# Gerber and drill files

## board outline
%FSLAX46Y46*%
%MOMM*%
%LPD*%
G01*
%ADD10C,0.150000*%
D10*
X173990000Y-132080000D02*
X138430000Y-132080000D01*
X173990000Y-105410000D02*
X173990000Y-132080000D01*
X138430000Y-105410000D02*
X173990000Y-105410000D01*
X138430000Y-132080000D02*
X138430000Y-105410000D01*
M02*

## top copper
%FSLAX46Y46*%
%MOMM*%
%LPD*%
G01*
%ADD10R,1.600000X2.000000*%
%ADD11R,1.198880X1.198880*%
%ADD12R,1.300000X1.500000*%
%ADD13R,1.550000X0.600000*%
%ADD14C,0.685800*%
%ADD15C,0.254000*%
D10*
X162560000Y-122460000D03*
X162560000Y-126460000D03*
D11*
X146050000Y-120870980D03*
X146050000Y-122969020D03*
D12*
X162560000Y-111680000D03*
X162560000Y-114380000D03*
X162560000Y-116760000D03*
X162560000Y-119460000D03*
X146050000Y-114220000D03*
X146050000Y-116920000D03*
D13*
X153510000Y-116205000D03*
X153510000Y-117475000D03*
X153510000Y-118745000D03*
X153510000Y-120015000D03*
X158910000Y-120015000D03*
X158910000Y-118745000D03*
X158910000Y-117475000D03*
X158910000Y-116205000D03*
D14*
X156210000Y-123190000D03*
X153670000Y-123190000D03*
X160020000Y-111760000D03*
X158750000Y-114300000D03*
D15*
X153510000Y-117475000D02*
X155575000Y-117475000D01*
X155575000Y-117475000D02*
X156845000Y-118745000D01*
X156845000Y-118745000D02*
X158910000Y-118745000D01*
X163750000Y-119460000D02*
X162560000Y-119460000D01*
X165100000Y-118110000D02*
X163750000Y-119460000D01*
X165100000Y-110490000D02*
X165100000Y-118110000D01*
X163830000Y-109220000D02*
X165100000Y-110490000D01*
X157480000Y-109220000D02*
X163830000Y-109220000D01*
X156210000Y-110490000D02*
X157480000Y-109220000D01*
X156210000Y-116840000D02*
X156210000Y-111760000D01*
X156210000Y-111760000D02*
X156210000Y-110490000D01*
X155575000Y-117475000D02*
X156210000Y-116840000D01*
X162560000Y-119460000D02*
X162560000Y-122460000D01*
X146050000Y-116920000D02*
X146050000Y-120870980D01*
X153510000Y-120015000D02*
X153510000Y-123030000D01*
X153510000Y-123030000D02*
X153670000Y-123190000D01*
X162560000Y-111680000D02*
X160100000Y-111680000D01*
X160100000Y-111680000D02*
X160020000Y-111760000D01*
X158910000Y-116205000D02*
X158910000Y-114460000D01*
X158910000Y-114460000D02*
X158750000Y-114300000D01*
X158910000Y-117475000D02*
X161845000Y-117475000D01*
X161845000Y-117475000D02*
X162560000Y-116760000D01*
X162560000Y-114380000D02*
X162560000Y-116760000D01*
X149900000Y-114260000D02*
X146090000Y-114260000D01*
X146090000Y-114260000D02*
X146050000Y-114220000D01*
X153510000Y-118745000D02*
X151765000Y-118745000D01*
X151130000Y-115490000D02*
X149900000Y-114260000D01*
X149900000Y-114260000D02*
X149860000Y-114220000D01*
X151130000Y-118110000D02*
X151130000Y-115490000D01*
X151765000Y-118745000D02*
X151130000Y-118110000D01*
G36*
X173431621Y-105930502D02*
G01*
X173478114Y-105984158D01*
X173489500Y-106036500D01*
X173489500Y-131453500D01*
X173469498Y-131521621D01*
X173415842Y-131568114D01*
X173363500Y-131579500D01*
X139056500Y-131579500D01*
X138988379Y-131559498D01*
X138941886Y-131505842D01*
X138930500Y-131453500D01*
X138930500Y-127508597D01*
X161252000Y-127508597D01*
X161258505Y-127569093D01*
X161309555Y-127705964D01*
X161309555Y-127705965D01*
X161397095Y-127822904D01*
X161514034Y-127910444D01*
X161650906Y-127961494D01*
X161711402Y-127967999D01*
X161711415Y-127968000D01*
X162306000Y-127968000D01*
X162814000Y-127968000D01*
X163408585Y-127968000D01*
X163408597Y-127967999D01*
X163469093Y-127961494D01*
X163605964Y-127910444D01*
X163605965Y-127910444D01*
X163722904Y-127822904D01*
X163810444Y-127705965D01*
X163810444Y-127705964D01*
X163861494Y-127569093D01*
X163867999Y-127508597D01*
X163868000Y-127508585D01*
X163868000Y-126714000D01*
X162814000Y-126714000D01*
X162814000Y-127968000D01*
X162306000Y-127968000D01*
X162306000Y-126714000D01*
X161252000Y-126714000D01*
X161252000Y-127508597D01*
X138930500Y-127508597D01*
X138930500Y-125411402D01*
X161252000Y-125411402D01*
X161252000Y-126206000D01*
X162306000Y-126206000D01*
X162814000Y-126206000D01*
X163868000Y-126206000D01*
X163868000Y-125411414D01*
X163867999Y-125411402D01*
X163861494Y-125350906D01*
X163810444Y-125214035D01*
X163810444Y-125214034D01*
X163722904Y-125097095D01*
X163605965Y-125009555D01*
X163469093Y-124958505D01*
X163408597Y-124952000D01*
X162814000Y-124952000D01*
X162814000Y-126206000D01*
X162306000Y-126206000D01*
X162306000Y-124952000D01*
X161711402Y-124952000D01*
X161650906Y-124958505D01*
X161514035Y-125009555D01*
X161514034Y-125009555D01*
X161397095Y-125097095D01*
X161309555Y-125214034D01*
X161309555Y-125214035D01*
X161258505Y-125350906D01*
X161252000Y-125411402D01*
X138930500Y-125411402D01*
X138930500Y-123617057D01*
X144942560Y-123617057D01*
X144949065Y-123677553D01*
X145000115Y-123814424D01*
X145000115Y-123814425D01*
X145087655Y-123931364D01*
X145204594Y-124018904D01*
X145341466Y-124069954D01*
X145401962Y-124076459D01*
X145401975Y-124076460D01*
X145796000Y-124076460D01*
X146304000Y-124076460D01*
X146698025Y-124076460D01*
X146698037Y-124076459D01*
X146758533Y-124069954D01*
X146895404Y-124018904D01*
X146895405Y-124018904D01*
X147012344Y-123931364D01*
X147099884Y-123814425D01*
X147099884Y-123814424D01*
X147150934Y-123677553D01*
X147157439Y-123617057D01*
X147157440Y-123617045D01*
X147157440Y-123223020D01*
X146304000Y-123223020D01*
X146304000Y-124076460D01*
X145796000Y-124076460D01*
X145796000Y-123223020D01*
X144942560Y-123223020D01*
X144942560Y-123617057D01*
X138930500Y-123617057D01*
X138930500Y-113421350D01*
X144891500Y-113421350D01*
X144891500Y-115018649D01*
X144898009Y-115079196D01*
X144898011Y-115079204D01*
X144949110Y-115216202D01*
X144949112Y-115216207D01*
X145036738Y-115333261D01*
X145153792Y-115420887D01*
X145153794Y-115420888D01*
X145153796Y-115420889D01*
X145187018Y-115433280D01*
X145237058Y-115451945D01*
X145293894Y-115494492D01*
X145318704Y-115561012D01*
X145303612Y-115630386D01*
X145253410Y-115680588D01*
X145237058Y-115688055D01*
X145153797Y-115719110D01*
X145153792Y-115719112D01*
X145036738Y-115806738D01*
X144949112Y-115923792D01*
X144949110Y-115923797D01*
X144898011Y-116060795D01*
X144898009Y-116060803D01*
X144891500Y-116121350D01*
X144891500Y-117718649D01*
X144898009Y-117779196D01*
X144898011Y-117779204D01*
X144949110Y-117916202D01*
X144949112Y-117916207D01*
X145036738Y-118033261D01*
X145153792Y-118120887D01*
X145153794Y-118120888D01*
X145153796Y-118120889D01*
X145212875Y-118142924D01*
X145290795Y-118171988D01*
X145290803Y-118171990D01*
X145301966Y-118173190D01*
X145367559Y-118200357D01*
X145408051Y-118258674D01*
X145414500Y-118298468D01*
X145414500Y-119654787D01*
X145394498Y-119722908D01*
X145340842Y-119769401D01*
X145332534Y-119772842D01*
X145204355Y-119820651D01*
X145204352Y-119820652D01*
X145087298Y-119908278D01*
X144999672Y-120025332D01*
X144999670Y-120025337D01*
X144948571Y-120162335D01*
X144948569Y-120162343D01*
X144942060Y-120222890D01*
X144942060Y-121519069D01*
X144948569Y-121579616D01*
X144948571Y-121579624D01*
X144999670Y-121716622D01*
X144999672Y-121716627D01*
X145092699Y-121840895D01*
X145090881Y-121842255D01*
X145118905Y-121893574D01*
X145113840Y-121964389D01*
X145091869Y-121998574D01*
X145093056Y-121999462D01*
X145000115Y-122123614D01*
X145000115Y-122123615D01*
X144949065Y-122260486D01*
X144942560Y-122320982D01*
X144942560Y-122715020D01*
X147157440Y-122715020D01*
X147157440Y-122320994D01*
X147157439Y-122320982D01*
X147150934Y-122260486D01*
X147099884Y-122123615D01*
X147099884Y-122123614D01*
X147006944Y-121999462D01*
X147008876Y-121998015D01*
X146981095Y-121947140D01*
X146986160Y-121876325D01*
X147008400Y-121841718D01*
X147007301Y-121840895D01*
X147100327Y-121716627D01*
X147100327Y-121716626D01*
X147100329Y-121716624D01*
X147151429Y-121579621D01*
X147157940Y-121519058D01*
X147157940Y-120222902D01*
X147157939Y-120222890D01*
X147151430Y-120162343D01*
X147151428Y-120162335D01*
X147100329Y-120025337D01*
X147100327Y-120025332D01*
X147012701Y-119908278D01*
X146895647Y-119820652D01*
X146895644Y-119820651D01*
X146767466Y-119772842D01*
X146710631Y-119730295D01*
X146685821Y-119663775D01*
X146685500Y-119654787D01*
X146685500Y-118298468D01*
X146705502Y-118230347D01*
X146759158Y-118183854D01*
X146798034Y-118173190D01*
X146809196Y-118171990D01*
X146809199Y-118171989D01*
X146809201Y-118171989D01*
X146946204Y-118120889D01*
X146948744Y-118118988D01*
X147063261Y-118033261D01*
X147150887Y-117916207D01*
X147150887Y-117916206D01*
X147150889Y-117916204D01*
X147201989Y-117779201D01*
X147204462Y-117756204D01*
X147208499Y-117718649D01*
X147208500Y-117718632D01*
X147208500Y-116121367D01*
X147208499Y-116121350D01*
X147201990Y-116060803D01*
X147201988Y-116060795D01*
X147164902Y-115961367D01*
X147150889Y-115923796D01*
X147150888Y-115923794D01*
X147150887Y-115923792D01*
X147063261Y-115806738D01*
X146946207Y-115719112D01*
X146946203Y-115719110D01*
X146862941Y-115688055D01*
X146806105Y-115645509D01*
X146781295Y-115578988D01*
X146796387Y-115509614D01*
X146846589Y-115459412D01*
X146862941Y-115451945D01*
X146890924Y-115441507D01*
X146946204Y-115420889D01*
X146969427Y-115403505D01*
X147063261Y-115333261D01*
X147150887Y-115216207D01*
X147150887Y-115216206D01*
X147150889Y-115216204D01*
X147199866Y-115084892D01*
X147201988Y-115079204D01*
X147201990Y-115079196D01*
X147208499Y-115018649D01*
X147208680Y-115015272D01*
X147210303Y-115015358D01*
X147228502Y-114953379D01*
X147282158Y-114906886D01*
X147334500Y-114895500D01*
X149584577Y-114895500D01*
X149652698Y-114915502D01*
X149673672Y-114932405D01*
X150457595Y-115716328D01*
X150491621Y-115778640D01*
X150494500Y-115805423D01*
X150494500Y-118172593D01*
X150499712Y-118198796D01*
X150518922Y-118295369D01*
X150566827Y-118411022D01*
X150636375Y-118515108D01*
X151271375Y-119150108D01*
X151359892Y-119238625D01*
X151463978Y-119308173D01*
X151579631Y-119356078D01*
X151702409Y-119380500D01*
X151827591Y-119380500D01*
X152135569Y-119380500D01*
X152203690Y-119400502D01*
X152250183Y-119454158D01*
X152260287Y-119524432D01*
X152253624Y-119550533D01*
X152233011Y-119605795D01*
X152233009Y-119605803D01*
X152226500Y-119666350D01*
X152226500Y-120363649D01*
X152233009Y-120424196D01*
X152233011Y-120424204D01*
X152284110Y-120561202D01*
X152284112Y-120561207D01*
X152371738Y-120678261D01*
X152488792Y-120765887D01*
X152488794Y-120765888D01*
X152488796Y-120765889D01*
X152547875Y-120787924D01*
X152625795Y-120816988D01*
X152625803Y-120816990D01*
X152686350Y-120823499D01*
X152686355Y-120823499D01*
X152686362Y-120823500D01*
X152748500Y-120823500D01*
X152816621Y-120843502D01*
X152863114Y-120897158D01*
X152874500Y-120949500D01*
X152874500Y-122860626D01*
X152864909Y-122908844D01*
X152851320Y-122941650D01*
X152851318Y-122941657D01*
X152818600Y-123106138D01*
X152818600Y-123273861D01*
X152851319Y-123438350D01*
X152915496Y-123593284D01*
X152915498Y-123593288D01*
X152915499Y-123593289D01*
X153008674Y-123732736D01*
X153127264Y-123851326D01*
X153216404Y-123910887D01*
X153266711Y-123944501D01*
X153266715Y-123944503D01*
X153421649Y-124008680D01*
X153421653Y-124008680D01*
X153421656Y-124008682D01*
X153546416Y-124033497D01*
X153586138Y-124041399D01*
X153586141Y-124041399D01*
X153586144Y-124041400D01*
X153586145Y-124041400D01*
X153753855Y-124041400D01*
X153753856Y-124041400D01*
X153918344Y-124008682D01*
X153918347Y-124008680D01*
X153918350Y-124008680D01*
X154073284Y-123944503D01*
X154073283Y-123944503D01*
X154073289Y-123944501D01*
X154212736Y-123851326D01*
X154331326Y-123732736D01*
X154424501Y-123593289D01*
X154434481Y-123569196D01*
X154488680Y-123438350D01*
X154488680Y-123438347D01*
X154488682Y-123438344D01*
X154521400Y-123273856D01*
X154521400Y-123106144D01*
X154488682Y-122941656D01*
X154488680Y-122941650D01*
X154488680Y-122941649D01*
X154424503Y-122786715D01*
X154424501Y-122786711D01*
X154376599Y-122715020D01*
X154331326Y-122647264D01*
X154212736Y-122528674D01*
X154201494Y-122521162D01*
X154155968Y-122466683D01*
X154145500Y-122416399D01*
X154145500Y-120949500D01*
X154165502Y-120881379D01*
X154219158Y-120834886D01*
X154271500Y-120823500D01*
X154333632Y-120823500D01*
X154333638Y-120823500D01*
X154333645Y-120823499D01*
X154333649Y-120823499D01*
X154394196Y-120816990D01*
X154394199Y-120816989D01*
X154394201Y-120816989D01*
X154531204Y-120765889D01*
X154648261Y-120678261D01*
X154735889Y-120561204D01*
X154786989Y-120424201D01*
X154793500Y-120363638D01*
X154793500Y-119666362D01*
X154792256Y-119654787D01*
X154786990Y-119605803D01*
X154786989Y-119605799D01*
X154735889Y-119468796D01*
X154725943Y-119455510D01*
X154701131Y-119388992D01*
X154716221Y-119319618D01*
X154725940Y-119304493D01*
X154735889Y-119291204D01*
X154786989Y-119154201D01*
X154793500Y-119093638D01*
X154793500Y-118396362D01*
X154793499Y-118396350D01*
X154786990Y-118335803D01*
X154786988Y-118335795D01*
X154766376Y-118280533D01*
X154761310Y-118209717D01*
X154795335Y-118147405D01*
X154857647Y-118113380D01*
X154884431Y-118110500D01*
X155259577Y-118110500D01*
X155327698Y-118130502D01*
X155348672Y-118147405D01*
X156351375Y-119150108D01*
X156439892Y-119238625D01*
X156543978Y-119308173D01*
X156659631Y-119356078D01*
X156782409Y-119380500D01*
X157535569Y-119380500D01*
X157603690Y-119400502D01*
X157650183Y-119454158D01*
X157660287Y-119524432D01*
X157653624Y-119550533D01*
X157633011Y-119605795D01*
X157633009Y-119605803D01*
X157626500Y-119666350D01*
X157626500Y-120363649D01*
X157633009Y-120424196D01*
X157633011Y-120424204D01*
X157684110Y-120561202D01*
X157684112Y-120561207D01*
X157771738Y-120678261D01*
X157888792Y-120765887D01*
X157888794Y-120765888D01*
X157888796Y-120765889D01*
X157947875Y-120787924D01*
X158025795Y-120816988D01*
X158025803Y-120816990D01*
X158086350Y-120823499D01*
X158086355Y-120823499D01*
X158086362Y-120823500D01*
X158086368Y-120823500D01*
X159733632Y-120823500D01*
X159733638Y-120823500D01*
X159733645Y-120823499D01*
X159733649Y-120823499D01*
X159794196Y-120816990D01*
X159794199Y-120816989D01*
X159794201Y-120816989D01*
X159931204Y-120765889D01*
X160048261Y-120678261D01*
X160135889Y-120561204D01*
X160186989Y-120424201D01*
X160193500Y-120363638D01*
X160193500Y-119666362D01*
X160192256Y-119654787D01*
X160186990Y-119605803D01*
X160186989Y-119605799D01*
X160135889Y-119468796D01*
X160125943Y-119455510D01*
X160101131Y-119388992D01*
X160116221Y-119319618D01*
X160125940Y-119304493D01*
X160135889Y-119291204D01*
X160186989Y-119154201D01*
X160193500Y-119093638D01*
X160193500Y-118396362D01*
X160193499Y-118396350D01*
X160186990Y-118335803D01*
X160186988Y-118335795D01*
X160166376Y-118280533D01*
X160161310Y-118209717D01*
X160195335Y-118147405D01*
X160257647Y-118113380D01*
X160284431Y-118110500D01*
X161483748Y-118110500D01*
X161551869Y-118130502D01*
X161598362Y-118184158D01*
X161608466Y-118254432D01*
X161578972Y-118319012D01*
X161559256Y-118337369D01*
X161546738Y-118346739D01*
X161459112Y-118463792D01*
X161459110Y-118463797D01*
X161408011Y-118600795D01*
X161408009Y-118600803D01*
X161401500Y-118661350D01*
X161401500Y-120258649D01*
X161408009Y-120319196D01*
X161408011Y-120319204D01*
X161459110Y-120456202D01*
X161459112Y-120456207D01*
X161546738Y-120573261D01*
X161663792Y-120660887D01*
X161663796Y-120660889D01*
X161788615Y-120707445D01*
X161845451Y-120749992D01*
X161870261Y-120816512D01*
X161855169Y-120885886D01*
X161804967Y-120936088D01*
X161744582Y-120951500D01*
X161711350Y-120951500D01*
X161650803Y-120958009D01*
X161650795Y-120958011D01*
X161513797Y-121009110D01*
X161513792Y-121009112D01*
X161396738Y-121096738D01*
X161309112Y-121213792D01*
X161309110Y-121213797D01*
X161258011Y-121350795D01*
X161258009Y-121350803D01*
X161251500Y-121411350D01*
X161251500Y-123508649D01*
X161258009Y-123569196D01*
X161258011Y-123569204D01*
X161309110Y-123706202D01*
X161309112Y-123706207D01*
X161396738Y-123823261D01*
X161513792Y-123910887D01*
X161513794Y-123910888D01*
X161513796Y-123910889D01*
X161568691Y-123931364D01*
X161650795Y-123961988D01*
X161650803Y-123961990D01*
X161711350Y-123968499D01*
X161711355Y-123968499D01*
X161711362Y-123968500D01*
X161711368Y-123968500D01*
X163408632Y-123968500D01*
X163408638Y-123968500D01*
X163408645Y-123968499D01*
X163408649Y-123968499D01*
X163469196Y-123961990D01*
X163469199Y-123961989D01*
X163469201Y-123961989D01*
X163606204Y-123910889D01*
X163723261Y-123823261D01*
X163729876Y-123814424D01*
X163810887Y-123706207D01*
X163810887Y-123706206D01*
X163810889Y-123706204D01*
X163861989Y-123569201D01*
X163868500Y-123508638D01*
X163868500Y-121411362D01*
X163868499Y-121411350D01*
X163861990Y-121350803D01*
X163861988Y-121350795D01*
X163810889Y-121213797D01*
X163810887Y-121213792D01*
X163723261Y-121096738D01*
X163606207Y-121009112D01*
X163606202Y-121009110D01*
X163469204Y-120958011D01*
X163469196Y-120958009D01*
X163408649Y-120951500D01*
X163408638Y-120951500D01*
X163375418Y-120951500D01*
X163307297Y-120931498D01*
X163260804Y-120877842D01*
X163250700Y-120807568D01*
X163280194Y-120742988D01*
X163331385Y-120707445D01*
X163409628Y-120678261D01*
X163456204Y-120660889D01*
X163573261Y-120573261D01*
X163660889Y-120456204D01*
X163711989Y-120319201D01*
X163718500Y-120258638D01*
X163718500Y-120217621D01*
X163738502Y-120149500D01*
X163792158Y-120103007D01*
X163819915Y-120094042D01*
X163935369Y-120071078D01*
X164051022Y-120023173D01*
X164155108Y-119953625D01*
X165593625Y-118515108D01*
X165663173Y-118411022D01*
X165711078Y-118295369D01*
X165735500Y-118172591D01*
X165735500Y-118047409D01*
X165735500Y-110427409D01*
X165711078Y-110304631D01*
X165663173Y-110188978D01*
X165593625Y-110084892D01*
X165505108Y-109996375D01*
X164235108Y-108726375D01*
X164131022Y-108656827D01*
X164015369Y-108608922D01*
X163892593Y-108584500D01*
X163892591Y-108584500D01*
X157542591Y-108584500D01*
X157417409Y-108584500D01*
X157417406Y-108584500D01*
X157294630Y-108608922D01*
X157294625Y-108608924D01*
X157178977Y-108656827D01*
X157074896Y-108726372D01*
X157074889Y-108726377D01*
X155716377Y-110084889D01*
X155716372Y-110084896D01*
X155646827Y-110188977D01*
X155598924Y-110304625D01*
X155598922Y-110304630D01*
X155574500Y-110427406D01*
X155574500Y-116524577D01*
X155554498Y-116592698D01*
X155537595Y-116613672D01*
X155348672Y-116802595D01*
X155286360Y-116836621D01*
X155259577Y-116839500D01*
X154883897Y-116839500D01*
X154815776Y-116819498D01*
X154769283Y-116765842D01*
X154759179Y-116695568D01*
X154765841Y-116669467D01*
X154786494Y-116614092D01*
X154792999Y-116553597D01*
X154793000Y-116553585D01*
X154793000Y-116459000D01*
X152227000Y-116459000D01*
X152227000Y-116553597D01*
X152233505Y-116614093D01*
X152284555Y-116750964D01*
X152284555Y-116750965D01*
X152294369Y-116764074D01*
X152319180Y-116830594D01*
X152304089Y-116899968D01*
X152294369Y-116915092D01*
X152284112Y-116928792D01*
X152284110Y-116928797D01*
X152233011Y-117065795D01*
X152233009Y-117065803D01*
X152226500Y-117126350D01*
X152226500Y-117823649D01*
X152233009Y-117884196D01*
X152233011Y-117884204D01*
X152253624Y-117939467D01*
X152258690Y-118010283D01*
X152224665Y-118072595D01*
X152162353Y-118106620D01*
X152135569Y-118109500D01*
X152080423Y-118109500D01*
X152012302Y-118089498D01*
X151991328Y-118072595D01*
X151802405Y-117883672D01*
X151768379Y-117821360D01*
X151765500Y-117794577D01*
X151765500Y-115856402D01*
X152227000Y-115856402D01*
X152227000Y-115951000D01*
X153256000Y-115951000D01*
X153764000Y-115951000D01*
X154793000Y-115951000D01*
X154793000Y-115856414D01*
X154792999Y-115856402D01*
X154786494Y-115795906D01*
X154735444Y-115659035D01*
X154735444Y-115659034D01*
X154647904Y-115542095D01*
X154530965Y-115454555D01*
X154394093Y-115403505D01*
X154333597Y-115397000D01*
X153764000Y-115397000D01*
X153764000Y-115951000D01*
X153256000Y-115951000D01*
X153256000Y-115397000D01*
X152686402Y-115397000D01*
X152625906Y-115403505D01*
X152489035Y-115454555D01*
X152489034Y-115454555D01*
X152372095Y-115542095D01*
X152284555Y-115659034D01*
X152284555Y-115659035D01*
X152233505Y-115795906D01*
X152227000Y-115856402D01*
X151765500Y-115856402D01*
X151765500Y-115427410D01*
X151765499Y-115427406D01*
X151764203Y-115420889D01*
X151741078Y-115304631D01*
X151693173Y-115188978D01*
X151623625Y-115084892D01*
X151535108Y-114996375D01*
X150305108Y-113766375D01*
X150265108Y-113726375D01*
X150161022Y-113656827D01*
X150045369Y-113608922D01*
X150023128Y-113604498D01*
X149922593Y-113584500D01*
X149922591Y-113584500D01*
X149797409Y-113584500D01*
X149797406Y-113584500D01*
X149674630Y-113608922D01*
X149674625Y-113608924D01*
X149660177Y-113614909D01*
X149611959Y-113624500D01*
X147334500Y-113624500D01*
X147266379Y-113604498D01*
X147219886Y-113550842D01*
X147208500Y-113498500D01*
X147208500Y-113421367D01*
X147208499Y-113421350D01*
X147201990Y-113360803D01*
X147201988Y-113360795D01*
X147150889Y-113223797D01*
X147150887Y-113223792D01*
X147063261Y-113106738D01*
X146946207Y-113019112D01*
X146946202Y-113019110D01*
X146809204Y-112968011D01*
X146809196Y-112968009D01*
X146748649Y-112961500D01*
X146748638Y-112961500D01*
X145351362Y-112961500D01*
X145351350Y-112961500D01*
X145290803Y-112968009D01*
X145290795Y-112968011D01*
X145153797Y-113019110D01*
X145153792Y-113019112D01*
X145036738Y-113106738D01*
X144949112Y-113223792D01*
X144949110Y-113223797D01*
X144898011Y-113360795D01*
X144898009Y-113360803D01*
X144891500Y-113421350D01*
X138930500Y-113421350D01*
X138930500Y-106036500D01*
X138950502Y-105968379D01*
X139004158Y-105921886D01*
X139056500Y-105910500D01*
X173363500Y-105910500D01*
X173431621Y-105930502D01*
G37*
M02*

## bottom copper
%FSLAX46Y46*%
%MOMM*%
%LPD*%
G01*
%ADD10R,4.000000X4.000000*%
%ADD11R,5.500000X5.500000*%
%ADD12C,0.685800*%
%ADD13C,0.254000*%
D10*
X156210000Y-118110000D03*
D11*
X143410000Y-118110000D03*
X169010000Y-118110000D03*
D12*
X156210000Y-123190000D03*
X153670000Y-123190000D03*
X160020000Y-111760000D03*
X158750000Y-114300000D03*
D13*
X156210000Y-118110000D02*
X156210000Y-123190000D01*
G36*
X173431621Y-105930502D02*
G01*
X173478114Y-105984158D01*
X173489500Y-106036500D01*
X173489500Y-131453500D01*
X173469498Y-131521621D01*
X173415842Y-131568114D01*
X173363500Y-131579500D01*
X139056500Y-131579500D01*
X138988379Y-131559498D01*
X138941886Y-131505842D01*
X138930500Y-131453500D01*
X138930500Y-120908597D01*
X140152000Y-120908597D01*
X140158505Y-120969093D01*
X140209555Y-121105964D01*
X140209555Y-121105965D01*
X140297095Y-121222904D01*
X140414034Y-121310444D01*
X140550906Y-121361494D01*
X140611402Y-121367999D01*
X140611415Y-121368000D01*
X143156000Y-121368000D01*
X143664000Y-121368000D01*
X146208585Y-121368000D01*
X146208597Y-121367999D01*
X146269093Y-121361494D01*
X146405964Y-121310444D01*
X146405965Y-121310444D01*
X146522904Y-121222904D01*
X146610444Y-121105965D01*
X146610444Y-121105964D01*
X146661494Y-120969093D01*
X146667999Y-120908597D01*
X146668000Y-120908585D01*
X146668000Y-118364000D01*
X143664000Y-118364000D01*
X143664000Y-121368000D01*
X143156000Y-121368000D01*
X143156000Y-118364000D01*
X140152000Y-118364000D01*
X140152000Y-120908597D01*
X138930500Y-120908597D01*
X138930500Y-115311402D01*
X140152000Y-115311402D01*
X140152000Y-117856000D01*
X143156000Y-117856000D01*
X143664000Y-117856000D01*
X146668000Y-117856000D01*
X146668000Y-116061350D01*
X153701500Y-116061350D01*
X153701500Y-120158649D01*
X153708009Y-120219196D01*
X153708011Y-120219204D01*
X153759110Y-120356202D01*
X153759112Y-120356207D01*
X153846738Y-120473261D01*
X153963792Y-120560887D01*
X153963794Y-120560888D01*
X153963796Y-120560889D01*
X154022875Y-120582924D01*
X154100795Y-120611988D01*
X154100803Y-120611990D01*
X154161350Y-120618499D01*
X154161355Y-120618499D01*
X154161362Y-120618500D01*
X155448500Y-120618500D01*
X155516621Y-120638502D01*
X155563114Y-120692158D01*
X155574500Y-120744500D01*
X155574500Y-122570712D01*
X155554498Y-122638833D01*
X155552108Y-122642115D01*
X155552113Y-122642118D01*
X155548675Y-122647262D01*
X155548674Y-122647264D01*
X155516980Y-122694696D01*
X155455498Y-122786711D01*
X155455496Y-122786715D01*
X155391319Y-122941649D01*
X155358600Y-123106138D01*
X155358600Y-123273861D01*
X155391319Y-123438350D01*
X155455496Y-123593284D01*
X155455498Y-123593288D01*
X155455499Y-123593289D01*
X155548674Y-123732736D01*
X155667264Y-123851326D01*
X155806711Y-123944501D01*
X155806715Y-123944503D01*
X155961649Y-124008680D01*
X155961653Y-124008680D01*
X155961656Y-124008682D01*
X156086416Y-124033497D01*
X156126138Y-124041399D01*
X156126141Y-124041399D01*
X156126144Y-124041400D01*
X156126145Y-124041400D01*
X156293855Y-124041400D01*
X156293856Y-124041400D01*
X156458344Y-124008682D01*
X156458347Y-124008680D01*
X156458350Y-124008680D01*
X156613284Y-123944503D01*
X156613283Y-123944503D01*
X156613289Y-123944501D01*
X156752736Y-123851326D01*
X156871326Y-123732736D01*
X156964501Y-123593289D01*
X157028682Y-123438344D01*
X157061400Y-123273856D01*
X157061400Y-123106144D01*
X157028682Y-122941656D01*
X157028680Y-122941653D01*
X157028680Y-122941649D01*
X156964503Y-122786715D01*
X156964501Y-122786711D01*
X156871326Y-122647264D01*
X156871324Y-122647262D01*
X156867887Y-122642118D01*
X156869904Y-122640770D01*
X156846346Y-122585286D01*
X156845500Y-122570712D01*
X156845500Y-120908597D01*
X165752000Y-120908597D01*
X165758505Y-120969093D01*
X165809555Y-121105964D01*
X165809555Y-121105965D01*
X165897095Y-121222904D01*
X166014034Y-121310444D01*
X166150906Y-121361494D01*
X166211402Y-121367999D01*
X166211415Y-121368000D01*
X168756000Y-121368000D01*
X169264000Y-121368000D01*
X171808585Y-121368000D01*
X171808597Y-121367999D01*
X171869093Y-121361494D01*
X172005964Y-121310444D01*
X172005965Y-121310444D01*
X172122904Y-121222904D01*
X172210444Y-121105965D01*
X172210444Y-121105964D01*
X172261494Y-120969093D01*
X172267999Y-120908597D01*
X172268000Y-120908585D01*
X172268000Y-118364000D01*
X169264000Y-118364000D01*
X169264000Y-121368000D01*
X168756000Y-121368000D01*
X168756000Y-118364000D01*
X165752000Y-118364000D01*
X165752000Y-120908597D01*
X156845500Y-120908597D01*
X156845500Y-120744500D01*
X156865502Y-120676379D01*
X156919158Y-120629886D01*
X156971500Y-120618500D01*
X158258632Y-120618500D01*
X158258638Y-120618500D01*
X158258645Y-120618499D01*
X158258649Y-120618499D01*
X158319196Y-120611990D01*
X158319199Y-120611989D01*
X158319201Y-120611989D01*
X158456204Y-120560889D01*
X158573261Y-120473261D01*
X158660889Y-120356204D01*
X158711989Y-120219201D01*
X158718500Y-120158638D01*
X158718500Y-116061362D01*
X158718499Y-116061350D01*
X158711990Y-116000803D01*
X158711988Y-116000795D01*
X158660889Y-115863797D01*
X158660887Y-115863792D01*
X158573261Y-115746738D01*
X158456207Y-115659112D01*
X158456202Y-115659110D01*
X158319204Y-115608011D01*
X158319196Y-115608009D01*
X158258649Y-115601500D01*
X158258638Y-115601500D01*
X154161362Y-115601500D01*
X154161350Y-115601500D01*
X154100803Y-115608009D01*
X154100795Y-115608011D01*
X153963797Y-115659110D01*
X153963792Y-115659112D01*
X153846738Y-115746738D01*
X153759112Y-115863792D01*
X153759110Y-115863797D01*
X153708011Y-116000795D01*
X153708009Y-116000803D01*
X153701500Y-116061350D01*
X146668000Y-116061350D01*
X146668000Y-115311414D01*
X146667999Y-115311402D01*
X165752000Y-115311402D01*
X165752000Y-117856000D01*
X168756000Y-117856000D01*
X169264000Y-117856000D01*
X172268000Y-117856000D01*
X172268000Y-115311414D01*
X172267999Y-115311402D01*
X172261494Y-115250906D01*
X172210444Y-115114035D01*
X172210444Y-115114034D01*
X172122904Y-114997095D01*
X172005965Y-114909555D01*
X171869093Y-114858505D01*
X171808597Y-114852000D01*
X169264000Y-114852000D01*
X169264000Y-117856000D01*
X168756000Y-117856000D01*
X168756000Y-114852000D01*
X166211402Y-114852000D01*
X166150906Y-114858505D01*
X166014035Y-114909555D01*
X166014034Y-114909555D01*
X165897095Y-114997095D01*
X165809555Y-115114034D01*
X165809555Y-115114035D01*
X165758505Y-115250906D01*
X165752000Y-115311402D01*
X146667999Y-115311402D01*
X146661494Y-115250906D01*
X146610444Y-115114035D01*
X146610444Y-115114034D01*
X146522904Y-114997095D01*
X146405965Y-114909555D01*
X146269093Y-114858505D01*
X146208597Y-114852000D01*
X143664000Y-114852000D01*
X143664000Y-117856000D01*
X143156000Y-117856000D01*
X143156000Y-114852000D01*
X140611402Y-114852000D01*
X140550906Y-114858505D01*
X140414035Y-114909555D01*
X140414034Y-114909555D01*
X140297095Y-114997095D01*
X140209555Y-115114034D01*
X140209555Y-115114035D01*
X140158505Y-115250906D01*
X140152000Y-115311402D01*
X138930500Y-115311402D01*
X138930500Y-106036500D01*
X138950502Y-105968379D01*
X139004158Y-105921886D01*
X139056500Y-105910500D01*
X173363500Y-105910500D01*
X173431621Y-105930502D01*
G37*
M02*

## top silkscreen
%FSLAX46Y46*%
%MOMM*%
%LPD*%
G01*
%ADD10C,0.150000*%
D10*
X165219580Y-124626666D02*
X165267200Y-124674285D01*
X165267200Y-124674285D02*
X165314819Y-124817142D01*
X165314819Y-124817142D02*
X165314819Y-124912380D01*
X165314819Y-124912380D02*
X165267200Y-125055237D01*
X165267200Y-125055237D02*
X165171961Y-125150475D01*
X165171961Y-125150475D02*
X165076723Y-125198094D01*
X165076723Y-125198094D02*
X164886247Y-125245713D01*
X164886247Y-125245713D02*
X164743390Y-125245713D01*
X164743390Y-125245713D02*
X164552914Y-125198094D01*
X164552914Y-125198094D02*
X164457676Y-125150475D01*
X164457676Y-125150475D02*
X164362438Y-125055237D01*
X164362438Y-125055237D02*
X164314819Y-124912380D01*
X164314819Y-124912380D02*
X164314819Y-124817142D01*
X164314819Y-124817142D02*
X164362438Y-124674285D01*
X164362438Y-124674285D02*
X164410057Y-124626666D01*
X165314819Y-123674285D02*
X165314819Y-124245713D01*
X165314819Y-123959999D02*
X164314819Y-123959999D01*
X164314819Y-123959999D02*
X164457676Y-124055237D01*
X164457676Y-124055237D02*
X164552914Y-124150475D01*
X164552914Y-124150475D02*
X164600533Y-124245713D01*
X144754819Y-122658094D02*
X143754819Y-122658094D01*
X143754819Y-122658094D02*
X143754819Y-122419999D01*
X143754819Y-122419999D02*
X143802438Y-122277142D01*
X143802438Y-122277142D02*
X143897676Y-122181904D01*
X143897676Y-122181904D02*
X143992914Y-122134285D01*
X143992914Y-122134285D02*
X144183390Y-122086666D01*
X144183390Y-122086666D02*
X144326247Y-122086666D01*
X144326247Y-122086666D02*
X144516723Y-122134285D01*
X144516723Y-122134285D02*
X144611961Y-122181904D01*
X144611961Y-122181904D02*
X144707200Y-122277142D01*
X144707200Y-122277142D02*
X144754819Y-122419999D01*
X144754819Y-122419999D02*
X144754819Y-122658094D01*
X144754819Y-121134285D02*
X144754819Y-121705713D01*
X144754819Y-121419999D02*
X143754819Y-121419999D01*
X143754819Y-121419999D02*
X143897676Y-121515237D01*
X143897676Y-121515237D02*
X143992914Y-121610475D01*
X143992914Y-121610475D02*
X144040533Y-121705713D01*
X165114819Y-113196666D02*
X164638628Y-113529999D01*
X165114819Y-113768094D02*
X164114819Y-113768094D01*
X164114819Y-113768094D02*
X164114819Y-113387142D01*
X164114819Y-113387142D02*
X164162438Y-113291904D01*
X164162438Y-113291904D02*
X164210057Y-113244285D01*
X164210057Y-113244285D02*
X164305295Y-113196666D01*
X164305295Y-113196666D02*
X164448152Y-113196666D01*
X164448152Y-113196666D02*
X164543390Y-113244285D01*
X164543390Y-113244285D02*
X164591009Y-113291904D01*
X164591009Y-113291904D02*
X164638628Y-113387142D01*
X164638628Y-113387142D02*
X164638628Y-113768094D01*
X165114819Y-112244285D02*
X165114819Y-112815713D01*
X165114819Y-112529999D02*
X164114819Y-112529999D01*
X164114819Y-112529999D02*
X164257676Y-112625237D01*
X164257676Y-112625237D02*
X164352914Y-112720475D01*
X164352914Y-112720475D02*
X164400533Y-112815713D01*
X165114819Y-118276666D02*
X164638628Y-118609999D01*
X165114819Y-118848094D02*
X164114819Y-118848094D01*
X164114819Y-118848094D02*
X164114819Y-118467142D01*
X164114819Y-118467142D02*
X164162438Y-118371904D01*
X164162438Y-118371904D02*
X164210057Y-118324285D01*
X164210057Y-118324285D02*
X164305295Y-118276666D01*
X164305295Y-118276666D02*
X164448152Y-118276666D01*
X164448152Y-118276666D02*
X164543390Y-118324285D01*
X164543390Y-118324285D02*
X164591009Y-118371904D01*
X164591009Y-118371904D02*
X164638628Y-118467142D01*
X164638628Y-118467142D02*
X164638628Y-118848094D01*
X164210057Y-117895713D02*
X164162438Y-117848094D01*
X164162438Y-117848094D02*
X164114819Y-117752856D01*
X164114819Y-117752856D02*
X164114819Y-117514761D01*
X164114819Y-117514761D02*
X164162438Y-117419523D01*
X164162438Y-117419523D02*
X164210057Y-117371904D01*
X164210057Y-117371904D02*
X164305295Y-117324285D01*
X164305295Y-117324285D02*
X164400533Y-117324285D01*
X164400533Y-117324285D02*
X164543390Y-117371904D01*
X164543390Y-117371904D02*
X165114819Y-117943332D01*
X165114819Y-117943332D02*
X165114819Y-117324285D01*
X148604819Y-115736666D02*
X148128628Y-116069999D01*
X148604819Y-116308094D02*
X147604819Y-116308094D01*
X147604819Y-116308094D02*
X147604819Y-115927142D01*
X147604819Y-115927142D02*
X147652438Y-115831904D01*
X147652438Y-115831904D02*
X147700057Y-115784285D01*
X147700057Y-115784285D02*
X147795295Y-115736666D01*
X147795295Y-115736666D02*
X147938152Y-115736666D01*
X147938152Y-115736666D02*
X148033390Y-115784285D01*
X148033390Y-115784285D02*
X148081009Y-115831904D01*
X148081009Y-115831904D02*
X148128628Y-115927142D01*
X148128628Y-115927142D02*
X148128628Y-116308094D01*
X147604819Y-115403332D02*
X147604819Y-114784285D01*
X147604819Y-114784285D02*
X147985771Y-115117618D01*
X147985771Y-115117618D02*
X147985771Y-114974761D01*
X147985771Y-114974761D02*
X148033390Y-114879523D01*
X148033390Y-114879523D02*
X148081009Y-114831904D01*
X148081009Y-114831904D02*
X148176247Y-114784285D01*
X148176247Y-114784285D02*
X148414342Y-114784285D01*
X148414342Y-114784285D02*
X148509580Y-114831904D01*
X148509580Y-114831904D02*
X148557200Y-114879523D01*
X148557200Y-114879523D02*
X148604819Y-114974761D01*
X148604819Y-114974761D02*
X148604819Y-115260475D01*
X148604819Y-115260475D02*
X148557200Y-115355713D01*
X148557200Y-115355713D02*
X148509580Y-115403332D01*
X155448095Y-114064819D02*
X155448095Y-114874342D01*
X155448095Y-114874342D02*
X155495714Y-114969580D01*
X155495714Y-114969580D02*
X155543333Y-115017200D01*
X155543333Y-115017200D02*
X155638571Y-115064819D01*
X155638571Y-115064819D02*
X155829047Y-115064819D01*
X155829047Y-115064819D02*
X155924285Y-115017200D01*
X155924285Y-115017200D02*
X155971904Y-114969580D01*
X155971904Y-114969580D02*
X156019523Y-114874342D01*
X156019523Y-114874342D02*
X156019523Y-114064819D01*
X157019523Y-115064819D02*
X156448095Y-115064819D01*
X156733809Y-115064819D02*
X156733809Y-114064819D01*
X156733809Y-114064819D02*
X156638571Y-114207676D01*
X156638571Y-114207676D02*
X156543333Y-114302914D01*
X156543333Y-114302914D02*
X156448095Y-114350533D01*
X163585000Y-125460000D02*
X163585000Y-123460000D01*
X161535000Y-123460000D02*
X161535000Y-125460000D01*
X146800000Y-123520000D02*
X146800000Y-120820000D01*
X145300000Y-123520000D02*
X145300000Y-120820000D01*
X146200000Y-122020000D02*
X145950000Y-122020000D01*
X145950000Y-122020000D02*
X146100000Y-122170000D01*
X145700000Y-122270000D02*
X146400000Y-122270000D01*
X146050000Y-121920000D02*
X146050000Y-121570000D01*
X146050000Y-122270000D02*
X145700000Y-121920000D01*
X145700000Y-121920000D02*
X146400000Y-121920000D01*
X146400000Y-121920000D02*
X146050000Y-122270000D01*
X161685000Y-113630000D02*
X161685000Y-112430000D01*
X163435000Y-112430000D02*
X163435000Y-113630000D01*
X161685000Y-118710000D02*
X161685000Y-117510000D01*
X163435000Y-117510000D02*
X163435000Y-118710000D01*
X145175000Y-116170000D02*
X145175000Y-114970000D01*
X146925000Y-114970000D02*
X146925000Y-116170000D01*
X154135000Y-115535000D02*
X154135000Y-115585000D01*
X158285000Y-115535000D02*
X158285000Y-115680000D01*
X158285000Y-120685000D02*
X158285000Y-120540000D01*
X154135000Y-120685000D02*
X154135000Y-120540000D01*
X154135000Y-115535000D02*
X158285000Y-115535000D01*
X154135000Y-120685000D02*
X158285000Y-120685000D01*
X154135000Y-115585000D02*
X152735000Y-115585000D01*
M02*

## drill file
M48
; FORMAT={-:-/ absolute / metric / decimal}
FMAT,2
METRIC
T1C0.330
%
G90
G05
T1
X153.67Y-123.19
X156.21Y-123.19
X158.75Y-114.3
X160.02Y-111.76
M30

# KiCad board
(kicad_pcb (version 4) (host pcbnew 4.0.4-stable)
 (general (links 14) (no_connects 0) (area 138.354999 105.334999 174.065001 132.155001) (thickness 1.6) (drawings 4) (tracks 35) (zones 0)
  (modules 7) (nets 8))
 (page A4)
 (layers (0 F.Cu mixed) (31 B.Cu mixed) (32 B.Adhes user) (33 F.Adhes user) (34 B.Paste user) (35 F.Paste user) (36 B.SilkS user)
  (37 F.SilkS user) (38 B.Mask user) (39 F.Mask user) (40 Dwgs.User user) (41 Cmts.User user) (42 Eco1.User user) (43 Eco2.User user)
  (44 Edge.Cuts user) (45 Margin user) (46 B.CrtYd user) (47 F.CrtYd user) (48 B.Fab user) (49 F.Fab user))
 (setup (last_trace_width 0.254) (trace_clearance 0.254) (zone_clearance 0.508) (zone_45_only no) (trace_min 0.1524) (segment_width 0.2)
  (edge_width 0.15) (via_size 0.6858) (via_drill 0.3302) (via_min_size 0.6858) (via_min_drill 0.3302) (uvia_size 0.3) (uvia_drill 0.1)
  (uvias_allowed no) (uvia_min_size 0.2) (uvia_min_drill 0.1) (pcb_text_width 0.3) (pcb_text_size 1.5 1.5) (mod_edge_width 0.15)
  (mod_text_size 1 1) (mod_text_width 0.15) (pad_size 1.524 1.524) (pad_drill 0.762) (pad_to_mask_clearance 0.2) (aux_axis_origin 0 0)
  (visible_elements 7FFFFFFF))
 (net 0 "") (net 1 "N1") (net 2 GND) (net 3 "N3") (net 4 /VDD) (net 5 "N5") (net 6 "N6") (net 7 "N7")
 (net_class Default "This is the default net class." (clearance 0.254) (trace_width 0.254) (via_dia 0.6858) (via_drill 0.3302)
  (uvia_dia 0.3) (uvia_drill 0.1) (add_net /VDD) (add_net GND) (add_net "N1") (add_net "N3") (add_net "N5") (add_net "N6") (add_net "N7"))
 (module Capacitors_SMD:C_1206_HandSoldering (layer F.Cu) (at 162.56 124.46 270)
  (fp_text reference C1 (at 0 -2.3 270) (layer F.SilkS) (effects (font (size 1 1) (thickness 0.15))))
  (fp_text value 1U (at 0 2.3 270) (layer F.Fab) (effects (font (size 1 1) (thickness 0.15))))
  (fp_line (start 1 -1.025) (end -1 -1.025) (layer F.SilkS) (width 0.15))
  (fp_line (start -1 1.025) (end 1 1.025) (layer F.SilkS) (width 0.15))
  (pad 1 smd rect (at -2 0 270) (size 2 1.6) (layers F.Cu F.Paste F.Mask) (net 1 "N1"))
  (pad 2 smd rect (at 2 0 270) (size 2 1.6) (layers F.Cu F.Paste F.Mask) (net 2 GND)))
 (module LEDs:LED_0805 (layer F.Cu) (at 146.05 121.92 90)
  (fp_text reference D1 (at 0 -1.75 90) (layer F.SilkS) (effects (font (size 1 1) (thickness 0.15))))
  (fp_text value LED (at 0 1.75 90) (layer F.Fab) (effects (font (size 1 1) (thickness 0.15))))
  (fp_line (start -1.6 0.75) (end 1.1 0.75) (layer F.SilkS) (width 0.15))
  (fp_line (start -1.6 -0.75) (end 1.1 -0.75) (layer F.SilkS) (width 0.15))
  (fp_line (start -0.1 0.15) (end -0.1 -0.1) (layer F.SilkS) (width 0.15))
  (fp_line (start -0.1 -0.1) (end -0.25 0.05) (layer F.SilkS) (width 0.15))
  (fp_line (start -0.35 -0.35) (end -0.35 0.35) (layer F.SilkS) (width 0.15))
  (fp_line (start 0 0) (end 0.35 0) (layer F.SilkS) (width 0.15))
  (fp_line (start -0.35 0) (end 0 -0.35) (layer F.SilkS) (width 0.15))
  (fp_line (start 0 -0.35) (end 0 0.35) (layer F.SilkS) (width 0.15))
  (fp_line (start 0 0.35) (end -0.35 0) (layer F.SilkS) (width 0.15))
  (pad 2 smd rect (at 1.04902 0 270) (size 1.19888 1.19888) (layers F.Cu F.Paste F.Mask) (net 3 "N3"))
  (pad 1 smd rect (at -1.04902 0 270) (size 1.19888 1.19888) (layers F.Cu F.Paste F.Mask) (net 2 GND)))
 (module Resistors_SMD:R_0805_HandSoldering (layer F.Cu) (at 162.56 113.03 270)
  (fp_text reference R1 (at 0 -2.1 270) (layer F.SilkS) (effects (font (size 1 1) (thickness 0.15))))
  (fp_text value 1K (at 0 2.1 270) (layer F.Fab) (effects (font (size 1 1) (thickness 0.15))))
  (fp_line (start 0.6 0.875) (end -0.6 0.875) (layer F.SilkS) (width 0.15))
  (fp_line (start -0.6 -0.875) (end 0.6 -0.875) (layer F.SilkS) (width 0.15))
  (pad 1 smd rect (at -1.35 0 270) (size 1.5 1.3) (layers F.Cu F.Paste F.Mask) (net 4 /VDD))
  (pad 2 smd rect (at 1.35 0 270) (size 1.5 1.3) (layers F.Cu F.Paste F.Mask) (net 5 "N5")))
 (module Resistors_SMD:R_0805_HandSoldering (layer F.Cu) (at 162.56 118.11 270)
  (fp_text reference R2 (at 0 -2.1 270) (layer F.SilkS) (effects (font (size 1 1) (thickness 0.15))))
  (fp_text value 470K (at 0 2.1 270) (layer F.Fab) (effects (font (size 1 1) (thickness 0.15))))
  (fp_line (start 0.6 0.875) (end -0.6 0.875) (layer F.SilkS) (width 0.15))
  (fp_line (start -0.6 -0.875) (end 0.6 -0.875) (layer F.SilkS) (width 0.15))
  (pad 1 smd rect (at -1.35 0 270) (size 1.5 1.3) (layers F.Cu F.Paste F.Mask) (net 5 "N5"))
  (pad 2 smd rect (at 1.35 0 270) (size 1.5 1.3) (layers F.Cu F.Paste F.Mask) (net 1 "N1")))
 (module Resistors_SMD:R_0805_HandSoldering (layer F.Cu) (at 146.05 115.57 270)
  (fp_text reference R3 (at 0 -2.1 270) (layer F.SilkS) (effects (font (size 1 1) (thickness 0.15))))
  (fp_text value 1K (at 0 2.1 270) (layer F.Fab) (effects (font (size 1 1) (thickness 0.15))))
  (fp_line (start 0.6 0.875) (end -0.6 0.875) (layer F.SilkS) (width 0.15))
  (fp_line (start -0.6 -0.875) (end 0.6 -0.875) (layer F.SilkS) (width 0.15))
  (pad 1 smd rect (at -1.35 0 270) (size 1.5 1.3) (layers F.Cu F.Paste F.Mask) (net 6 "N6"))
  (pad 2 smd rect (at 1.35 0 270) (size 1.5 1.3) (layers F.Cu F.Paste F.Mask) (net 3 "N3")))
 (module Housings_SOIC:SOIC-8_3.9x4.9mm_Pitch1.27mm (layer F.Cu) (at 156.21 118.11)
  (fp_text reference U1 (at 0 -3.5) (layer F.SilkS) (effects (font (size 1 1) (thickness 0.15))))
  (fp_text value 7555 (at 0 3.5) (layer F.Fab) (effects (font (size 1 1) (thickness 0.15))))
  (fp_line (start -2.075 -2.575) (end -2.075 -2.525) (layer F.SilkS) (width 0.15))
  (fp_line (start 2.075 -2.575) (end 2.075 -2.43) (layer F.SilkS) (width 0.15))
  (fp_line (start 2.075 2.575) (end 2.075 2.43) (layer F.SilkS) (width 0.15))
  (fp_line (start -2.075 2.575) (end -2.075 2.43) (layer F.SilkS) (width 0.15))
  (fp_line (start -2.075 -2.575) (end 2.075 -2.575) (layer F.SilkS) (width 0.15))
  (fp_line (start -2.075 2.575) (end 2.075 2.575) (layer F.SilkS) (width 0.15))
  (fp_line (start -2.075 -2.525) (end -3.475 -2.525) (layer F.SilkS) (width 0.15))
  (pad 1 smd rect (at -2.7 -1.905) (size 1.55 0.6) (layers F.Cu F.Paste F.Mask) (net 2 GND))
  (pad 2 smd rect (at -2.7 -0.635) (size 1.55 0.6) (layers F.Cu F.Paste F.Mask) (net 1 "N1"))
  (pad 3 smd rect (at -2.7 0.635) (size 1.55 0.6) (layers F.Cu F.Paste F.Mask) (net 6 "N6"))
  (pad 4 smd rect (at -2.7 1.905) (size 1.55 0.6) (layers F.Cu F.Paste F.Mask) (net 4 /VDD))
  (pad 5 smd rect (at 2.7 1.905) (size 1.55 0.6) (layers F.Cu F.Paste F.Mask) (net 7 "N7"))
  (pad 6 smd rect (at 2.7 0.635) (size 1.55 0.6) (layers F.Cu F.Paste F.Mask) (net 1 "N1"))
  (pad 7 smd rect (at 2.7 -0.635) (size 1.55 0.6) (layers F.Cu F.Paste F.Mask) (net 5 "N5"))
  (pad 8 smd rect (at 2.7 -1.905) (size 1.55 0.6) (layers F.Cu F.Paste F.Mask) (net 4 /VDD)))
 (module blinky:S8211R (layer B.Cu) (at 156.21 118.11)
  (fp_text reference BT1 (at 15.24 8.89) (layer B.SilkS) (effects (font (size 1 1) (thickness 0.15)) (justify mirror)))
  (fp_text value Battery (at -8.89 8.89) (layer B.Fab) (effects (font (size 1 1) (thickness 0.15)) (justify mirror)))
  (pad 2 smd rect (at 0 0) (size 4 4) (layers B.Cu B.Paste B.Mask) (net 2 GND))
  (pad 1 smd rect (at -12.8 0) (size 5.5 5.5) (layers B.Cu B.Paste B.Mask) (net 4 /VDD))
  (pad 1 smd rect (at 12.8 0) (size 5.5 5.5) (layers B.Cu B.Paste B.Mask) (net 4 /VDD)))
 (gr_line (start 173.99 132.08) (end 138.43 132.08) (angle 90) (layer Edge.Cuts) (width 0.15))
 (gr_line (start 173.99 105.41) (end 173.99 132.08) (angle 90) (layer Edge.Cuts) (width 0.15))
 (gr_line (start 138.43 105.41) (end 173.99 105.41) (angle 90) (layer Edge.Cuts) (width 0.15))
 (gr_line (start 138.43 132.08) (end 138.43 105.41) (angle 90) (layer Edge.Cuts) (width 0.15))
 (segment (start 153.51 117.475) (end 155.575 117.475) (width 0.254) (layer F.Cu) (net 1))
 (segment (start 155.575 117.475) (end 156.845 118.745) (width 0.254) (layer F.Cu) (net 1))
 (segment (start 156.845 118.745) (end 158.91 118.745) (width 0.254) (layer F.Cu) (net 1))
 (segment (start 163.75 119.46) (end 162.56 119.46) (width 0.254) (layer F.Cu) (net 1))
 (segment (start 165.1 118.11) (end 163.75 119.46) (width 0.254) (layer F.Cu) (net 1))
 (segment (start 165.1 110.49) (end 165.1 118.11) (width 0.254) (layer F.Cu) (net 1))
 (segment (start 163.83 109.22) (end 165.1 110.49) (width 0.254) (layer F.Cu) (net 1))
 (segment (start 157.48 109.22) (end 163.83 109.22) (width 0.254) (layer F.Cu) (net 1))
 (segment (start 156.21 110.49) (end 157.48 109.22) (width 0.254) (layer F.Cu) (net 1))
 (segment (start 156.21 116.84) (end 156.21 111.76) (width 0.254) (layer F.Cu) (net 1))
 (segment (start 156.21 111.76) (end 156.21 110.49) (width 0.254) (layer F.Cu) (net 1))
 (segment (start 155.575 117.475) (end 156.21 116.84) (width 0.254) (layer F.Cu) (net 1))
 (segment (start 162.56 119.46) (end 162.56 122.46) (width 0.254) (layer F.Cu) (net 1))
 (segment (start 156.21 118.11) (end 156.21 123.19) (width 0.254) (layer B.Cu) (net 2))
 (via (at 156.21 123.19) (size 0.6858) (drill 0.3302) (layers F.Cu B.Cu) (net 2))
 (segment (start 146.05 116.92) (end 146.05 120.87098) (width 0.254) (layer F.Cu) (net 3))
 (segment (start 153.51 120.015) (end 153.51 123.03) (width 0.254) (layer F.Cu) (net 4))
 (via (at 153.67 123.19) (size 0.6858) (drill 0.3302) (layers F.Cu B.Cu) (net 4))
 (segment (start 153.51 123.03) (end 153.67 123.19) (width 0.254) (layer F.Cu) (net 4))
 (segment (start 162.56 111.68) (end 160.1 111.68) (width 0.254) (layer F.Cu) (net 4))
 (via (at 160.02 111.76) (size 0.6858) (drill 0.3302) (layers F.Cu B.Cu) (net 4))
 (segment (start 160.1 111.68) (end 160.02 111.76) (width 0.254) (layer F.Cu) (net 4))
 (segment (start 158.91 116.205) (end 158.91 114.46) (width 0.254) (layer F.Cu) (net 4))
 (via (at 158.75 114.3) (size 0.6858) (drill 0.3302) (layers F.Cu B.Cu) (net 4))
 (segment (start 158.91 114.46) (end 158.75 114.3) (width 0.254) (layer F.Cu) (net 4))
 (segment (start 158.91 117.475) (end 161.845 117.475) (width 0.254) (layer F.Cu) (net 5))
 (segment (start 161.845 117.475) (end 162.56 116.76) (width 0.254) (layer F.Cu) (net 5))
 (segment (start 162.56 114.38) (end 162.56 116.76) (width 0.254) (layer F.Cu) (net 5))
 (segment (start 149.9 114.26) (end 146.09 114.26) (width 0.254) (layer F.Cu) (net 6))
 (segment (start 146.09 114.26) (end 146.05 114.22) (width 0.254) (layer F.Cu) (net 6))
 (segment (start 153.51 118.745) (end 151.765 118.745) (width 0.254) (layer F.Cu) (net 6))
 (segment (start 151.13 115.49) (end 149.9 114.26) (width 0.254) (layer F.Cu) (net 6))
 (segment (start 149.9 114.26) (end 149.86 114.22) (width 0.254) (layer F.Cu) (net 6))
 (segment (start 151.13 118.11) (end 151.13 115.49) (width 0.254) (layer F.Cu) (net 6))
 (segment (start 151.765 118.745) (end 151.13 118.11) (width 0.254) (layer F.Cu) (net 6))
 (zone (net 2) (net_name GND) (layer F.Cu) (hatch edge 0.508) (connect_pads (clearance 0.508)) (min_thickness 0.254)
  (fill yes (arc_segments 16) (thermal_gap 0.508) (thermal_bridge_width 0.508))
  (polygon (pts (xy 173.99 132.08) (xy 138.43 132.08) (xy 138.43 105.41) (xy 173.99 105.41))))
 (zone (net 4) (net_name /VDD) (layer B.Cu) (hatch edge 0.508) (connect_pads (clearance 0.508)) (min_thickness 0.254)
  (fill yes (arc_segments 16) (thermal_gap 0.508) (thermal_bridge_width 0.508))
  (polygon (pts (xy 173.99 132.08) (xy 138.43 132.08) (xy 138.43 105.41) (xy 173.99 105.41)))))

